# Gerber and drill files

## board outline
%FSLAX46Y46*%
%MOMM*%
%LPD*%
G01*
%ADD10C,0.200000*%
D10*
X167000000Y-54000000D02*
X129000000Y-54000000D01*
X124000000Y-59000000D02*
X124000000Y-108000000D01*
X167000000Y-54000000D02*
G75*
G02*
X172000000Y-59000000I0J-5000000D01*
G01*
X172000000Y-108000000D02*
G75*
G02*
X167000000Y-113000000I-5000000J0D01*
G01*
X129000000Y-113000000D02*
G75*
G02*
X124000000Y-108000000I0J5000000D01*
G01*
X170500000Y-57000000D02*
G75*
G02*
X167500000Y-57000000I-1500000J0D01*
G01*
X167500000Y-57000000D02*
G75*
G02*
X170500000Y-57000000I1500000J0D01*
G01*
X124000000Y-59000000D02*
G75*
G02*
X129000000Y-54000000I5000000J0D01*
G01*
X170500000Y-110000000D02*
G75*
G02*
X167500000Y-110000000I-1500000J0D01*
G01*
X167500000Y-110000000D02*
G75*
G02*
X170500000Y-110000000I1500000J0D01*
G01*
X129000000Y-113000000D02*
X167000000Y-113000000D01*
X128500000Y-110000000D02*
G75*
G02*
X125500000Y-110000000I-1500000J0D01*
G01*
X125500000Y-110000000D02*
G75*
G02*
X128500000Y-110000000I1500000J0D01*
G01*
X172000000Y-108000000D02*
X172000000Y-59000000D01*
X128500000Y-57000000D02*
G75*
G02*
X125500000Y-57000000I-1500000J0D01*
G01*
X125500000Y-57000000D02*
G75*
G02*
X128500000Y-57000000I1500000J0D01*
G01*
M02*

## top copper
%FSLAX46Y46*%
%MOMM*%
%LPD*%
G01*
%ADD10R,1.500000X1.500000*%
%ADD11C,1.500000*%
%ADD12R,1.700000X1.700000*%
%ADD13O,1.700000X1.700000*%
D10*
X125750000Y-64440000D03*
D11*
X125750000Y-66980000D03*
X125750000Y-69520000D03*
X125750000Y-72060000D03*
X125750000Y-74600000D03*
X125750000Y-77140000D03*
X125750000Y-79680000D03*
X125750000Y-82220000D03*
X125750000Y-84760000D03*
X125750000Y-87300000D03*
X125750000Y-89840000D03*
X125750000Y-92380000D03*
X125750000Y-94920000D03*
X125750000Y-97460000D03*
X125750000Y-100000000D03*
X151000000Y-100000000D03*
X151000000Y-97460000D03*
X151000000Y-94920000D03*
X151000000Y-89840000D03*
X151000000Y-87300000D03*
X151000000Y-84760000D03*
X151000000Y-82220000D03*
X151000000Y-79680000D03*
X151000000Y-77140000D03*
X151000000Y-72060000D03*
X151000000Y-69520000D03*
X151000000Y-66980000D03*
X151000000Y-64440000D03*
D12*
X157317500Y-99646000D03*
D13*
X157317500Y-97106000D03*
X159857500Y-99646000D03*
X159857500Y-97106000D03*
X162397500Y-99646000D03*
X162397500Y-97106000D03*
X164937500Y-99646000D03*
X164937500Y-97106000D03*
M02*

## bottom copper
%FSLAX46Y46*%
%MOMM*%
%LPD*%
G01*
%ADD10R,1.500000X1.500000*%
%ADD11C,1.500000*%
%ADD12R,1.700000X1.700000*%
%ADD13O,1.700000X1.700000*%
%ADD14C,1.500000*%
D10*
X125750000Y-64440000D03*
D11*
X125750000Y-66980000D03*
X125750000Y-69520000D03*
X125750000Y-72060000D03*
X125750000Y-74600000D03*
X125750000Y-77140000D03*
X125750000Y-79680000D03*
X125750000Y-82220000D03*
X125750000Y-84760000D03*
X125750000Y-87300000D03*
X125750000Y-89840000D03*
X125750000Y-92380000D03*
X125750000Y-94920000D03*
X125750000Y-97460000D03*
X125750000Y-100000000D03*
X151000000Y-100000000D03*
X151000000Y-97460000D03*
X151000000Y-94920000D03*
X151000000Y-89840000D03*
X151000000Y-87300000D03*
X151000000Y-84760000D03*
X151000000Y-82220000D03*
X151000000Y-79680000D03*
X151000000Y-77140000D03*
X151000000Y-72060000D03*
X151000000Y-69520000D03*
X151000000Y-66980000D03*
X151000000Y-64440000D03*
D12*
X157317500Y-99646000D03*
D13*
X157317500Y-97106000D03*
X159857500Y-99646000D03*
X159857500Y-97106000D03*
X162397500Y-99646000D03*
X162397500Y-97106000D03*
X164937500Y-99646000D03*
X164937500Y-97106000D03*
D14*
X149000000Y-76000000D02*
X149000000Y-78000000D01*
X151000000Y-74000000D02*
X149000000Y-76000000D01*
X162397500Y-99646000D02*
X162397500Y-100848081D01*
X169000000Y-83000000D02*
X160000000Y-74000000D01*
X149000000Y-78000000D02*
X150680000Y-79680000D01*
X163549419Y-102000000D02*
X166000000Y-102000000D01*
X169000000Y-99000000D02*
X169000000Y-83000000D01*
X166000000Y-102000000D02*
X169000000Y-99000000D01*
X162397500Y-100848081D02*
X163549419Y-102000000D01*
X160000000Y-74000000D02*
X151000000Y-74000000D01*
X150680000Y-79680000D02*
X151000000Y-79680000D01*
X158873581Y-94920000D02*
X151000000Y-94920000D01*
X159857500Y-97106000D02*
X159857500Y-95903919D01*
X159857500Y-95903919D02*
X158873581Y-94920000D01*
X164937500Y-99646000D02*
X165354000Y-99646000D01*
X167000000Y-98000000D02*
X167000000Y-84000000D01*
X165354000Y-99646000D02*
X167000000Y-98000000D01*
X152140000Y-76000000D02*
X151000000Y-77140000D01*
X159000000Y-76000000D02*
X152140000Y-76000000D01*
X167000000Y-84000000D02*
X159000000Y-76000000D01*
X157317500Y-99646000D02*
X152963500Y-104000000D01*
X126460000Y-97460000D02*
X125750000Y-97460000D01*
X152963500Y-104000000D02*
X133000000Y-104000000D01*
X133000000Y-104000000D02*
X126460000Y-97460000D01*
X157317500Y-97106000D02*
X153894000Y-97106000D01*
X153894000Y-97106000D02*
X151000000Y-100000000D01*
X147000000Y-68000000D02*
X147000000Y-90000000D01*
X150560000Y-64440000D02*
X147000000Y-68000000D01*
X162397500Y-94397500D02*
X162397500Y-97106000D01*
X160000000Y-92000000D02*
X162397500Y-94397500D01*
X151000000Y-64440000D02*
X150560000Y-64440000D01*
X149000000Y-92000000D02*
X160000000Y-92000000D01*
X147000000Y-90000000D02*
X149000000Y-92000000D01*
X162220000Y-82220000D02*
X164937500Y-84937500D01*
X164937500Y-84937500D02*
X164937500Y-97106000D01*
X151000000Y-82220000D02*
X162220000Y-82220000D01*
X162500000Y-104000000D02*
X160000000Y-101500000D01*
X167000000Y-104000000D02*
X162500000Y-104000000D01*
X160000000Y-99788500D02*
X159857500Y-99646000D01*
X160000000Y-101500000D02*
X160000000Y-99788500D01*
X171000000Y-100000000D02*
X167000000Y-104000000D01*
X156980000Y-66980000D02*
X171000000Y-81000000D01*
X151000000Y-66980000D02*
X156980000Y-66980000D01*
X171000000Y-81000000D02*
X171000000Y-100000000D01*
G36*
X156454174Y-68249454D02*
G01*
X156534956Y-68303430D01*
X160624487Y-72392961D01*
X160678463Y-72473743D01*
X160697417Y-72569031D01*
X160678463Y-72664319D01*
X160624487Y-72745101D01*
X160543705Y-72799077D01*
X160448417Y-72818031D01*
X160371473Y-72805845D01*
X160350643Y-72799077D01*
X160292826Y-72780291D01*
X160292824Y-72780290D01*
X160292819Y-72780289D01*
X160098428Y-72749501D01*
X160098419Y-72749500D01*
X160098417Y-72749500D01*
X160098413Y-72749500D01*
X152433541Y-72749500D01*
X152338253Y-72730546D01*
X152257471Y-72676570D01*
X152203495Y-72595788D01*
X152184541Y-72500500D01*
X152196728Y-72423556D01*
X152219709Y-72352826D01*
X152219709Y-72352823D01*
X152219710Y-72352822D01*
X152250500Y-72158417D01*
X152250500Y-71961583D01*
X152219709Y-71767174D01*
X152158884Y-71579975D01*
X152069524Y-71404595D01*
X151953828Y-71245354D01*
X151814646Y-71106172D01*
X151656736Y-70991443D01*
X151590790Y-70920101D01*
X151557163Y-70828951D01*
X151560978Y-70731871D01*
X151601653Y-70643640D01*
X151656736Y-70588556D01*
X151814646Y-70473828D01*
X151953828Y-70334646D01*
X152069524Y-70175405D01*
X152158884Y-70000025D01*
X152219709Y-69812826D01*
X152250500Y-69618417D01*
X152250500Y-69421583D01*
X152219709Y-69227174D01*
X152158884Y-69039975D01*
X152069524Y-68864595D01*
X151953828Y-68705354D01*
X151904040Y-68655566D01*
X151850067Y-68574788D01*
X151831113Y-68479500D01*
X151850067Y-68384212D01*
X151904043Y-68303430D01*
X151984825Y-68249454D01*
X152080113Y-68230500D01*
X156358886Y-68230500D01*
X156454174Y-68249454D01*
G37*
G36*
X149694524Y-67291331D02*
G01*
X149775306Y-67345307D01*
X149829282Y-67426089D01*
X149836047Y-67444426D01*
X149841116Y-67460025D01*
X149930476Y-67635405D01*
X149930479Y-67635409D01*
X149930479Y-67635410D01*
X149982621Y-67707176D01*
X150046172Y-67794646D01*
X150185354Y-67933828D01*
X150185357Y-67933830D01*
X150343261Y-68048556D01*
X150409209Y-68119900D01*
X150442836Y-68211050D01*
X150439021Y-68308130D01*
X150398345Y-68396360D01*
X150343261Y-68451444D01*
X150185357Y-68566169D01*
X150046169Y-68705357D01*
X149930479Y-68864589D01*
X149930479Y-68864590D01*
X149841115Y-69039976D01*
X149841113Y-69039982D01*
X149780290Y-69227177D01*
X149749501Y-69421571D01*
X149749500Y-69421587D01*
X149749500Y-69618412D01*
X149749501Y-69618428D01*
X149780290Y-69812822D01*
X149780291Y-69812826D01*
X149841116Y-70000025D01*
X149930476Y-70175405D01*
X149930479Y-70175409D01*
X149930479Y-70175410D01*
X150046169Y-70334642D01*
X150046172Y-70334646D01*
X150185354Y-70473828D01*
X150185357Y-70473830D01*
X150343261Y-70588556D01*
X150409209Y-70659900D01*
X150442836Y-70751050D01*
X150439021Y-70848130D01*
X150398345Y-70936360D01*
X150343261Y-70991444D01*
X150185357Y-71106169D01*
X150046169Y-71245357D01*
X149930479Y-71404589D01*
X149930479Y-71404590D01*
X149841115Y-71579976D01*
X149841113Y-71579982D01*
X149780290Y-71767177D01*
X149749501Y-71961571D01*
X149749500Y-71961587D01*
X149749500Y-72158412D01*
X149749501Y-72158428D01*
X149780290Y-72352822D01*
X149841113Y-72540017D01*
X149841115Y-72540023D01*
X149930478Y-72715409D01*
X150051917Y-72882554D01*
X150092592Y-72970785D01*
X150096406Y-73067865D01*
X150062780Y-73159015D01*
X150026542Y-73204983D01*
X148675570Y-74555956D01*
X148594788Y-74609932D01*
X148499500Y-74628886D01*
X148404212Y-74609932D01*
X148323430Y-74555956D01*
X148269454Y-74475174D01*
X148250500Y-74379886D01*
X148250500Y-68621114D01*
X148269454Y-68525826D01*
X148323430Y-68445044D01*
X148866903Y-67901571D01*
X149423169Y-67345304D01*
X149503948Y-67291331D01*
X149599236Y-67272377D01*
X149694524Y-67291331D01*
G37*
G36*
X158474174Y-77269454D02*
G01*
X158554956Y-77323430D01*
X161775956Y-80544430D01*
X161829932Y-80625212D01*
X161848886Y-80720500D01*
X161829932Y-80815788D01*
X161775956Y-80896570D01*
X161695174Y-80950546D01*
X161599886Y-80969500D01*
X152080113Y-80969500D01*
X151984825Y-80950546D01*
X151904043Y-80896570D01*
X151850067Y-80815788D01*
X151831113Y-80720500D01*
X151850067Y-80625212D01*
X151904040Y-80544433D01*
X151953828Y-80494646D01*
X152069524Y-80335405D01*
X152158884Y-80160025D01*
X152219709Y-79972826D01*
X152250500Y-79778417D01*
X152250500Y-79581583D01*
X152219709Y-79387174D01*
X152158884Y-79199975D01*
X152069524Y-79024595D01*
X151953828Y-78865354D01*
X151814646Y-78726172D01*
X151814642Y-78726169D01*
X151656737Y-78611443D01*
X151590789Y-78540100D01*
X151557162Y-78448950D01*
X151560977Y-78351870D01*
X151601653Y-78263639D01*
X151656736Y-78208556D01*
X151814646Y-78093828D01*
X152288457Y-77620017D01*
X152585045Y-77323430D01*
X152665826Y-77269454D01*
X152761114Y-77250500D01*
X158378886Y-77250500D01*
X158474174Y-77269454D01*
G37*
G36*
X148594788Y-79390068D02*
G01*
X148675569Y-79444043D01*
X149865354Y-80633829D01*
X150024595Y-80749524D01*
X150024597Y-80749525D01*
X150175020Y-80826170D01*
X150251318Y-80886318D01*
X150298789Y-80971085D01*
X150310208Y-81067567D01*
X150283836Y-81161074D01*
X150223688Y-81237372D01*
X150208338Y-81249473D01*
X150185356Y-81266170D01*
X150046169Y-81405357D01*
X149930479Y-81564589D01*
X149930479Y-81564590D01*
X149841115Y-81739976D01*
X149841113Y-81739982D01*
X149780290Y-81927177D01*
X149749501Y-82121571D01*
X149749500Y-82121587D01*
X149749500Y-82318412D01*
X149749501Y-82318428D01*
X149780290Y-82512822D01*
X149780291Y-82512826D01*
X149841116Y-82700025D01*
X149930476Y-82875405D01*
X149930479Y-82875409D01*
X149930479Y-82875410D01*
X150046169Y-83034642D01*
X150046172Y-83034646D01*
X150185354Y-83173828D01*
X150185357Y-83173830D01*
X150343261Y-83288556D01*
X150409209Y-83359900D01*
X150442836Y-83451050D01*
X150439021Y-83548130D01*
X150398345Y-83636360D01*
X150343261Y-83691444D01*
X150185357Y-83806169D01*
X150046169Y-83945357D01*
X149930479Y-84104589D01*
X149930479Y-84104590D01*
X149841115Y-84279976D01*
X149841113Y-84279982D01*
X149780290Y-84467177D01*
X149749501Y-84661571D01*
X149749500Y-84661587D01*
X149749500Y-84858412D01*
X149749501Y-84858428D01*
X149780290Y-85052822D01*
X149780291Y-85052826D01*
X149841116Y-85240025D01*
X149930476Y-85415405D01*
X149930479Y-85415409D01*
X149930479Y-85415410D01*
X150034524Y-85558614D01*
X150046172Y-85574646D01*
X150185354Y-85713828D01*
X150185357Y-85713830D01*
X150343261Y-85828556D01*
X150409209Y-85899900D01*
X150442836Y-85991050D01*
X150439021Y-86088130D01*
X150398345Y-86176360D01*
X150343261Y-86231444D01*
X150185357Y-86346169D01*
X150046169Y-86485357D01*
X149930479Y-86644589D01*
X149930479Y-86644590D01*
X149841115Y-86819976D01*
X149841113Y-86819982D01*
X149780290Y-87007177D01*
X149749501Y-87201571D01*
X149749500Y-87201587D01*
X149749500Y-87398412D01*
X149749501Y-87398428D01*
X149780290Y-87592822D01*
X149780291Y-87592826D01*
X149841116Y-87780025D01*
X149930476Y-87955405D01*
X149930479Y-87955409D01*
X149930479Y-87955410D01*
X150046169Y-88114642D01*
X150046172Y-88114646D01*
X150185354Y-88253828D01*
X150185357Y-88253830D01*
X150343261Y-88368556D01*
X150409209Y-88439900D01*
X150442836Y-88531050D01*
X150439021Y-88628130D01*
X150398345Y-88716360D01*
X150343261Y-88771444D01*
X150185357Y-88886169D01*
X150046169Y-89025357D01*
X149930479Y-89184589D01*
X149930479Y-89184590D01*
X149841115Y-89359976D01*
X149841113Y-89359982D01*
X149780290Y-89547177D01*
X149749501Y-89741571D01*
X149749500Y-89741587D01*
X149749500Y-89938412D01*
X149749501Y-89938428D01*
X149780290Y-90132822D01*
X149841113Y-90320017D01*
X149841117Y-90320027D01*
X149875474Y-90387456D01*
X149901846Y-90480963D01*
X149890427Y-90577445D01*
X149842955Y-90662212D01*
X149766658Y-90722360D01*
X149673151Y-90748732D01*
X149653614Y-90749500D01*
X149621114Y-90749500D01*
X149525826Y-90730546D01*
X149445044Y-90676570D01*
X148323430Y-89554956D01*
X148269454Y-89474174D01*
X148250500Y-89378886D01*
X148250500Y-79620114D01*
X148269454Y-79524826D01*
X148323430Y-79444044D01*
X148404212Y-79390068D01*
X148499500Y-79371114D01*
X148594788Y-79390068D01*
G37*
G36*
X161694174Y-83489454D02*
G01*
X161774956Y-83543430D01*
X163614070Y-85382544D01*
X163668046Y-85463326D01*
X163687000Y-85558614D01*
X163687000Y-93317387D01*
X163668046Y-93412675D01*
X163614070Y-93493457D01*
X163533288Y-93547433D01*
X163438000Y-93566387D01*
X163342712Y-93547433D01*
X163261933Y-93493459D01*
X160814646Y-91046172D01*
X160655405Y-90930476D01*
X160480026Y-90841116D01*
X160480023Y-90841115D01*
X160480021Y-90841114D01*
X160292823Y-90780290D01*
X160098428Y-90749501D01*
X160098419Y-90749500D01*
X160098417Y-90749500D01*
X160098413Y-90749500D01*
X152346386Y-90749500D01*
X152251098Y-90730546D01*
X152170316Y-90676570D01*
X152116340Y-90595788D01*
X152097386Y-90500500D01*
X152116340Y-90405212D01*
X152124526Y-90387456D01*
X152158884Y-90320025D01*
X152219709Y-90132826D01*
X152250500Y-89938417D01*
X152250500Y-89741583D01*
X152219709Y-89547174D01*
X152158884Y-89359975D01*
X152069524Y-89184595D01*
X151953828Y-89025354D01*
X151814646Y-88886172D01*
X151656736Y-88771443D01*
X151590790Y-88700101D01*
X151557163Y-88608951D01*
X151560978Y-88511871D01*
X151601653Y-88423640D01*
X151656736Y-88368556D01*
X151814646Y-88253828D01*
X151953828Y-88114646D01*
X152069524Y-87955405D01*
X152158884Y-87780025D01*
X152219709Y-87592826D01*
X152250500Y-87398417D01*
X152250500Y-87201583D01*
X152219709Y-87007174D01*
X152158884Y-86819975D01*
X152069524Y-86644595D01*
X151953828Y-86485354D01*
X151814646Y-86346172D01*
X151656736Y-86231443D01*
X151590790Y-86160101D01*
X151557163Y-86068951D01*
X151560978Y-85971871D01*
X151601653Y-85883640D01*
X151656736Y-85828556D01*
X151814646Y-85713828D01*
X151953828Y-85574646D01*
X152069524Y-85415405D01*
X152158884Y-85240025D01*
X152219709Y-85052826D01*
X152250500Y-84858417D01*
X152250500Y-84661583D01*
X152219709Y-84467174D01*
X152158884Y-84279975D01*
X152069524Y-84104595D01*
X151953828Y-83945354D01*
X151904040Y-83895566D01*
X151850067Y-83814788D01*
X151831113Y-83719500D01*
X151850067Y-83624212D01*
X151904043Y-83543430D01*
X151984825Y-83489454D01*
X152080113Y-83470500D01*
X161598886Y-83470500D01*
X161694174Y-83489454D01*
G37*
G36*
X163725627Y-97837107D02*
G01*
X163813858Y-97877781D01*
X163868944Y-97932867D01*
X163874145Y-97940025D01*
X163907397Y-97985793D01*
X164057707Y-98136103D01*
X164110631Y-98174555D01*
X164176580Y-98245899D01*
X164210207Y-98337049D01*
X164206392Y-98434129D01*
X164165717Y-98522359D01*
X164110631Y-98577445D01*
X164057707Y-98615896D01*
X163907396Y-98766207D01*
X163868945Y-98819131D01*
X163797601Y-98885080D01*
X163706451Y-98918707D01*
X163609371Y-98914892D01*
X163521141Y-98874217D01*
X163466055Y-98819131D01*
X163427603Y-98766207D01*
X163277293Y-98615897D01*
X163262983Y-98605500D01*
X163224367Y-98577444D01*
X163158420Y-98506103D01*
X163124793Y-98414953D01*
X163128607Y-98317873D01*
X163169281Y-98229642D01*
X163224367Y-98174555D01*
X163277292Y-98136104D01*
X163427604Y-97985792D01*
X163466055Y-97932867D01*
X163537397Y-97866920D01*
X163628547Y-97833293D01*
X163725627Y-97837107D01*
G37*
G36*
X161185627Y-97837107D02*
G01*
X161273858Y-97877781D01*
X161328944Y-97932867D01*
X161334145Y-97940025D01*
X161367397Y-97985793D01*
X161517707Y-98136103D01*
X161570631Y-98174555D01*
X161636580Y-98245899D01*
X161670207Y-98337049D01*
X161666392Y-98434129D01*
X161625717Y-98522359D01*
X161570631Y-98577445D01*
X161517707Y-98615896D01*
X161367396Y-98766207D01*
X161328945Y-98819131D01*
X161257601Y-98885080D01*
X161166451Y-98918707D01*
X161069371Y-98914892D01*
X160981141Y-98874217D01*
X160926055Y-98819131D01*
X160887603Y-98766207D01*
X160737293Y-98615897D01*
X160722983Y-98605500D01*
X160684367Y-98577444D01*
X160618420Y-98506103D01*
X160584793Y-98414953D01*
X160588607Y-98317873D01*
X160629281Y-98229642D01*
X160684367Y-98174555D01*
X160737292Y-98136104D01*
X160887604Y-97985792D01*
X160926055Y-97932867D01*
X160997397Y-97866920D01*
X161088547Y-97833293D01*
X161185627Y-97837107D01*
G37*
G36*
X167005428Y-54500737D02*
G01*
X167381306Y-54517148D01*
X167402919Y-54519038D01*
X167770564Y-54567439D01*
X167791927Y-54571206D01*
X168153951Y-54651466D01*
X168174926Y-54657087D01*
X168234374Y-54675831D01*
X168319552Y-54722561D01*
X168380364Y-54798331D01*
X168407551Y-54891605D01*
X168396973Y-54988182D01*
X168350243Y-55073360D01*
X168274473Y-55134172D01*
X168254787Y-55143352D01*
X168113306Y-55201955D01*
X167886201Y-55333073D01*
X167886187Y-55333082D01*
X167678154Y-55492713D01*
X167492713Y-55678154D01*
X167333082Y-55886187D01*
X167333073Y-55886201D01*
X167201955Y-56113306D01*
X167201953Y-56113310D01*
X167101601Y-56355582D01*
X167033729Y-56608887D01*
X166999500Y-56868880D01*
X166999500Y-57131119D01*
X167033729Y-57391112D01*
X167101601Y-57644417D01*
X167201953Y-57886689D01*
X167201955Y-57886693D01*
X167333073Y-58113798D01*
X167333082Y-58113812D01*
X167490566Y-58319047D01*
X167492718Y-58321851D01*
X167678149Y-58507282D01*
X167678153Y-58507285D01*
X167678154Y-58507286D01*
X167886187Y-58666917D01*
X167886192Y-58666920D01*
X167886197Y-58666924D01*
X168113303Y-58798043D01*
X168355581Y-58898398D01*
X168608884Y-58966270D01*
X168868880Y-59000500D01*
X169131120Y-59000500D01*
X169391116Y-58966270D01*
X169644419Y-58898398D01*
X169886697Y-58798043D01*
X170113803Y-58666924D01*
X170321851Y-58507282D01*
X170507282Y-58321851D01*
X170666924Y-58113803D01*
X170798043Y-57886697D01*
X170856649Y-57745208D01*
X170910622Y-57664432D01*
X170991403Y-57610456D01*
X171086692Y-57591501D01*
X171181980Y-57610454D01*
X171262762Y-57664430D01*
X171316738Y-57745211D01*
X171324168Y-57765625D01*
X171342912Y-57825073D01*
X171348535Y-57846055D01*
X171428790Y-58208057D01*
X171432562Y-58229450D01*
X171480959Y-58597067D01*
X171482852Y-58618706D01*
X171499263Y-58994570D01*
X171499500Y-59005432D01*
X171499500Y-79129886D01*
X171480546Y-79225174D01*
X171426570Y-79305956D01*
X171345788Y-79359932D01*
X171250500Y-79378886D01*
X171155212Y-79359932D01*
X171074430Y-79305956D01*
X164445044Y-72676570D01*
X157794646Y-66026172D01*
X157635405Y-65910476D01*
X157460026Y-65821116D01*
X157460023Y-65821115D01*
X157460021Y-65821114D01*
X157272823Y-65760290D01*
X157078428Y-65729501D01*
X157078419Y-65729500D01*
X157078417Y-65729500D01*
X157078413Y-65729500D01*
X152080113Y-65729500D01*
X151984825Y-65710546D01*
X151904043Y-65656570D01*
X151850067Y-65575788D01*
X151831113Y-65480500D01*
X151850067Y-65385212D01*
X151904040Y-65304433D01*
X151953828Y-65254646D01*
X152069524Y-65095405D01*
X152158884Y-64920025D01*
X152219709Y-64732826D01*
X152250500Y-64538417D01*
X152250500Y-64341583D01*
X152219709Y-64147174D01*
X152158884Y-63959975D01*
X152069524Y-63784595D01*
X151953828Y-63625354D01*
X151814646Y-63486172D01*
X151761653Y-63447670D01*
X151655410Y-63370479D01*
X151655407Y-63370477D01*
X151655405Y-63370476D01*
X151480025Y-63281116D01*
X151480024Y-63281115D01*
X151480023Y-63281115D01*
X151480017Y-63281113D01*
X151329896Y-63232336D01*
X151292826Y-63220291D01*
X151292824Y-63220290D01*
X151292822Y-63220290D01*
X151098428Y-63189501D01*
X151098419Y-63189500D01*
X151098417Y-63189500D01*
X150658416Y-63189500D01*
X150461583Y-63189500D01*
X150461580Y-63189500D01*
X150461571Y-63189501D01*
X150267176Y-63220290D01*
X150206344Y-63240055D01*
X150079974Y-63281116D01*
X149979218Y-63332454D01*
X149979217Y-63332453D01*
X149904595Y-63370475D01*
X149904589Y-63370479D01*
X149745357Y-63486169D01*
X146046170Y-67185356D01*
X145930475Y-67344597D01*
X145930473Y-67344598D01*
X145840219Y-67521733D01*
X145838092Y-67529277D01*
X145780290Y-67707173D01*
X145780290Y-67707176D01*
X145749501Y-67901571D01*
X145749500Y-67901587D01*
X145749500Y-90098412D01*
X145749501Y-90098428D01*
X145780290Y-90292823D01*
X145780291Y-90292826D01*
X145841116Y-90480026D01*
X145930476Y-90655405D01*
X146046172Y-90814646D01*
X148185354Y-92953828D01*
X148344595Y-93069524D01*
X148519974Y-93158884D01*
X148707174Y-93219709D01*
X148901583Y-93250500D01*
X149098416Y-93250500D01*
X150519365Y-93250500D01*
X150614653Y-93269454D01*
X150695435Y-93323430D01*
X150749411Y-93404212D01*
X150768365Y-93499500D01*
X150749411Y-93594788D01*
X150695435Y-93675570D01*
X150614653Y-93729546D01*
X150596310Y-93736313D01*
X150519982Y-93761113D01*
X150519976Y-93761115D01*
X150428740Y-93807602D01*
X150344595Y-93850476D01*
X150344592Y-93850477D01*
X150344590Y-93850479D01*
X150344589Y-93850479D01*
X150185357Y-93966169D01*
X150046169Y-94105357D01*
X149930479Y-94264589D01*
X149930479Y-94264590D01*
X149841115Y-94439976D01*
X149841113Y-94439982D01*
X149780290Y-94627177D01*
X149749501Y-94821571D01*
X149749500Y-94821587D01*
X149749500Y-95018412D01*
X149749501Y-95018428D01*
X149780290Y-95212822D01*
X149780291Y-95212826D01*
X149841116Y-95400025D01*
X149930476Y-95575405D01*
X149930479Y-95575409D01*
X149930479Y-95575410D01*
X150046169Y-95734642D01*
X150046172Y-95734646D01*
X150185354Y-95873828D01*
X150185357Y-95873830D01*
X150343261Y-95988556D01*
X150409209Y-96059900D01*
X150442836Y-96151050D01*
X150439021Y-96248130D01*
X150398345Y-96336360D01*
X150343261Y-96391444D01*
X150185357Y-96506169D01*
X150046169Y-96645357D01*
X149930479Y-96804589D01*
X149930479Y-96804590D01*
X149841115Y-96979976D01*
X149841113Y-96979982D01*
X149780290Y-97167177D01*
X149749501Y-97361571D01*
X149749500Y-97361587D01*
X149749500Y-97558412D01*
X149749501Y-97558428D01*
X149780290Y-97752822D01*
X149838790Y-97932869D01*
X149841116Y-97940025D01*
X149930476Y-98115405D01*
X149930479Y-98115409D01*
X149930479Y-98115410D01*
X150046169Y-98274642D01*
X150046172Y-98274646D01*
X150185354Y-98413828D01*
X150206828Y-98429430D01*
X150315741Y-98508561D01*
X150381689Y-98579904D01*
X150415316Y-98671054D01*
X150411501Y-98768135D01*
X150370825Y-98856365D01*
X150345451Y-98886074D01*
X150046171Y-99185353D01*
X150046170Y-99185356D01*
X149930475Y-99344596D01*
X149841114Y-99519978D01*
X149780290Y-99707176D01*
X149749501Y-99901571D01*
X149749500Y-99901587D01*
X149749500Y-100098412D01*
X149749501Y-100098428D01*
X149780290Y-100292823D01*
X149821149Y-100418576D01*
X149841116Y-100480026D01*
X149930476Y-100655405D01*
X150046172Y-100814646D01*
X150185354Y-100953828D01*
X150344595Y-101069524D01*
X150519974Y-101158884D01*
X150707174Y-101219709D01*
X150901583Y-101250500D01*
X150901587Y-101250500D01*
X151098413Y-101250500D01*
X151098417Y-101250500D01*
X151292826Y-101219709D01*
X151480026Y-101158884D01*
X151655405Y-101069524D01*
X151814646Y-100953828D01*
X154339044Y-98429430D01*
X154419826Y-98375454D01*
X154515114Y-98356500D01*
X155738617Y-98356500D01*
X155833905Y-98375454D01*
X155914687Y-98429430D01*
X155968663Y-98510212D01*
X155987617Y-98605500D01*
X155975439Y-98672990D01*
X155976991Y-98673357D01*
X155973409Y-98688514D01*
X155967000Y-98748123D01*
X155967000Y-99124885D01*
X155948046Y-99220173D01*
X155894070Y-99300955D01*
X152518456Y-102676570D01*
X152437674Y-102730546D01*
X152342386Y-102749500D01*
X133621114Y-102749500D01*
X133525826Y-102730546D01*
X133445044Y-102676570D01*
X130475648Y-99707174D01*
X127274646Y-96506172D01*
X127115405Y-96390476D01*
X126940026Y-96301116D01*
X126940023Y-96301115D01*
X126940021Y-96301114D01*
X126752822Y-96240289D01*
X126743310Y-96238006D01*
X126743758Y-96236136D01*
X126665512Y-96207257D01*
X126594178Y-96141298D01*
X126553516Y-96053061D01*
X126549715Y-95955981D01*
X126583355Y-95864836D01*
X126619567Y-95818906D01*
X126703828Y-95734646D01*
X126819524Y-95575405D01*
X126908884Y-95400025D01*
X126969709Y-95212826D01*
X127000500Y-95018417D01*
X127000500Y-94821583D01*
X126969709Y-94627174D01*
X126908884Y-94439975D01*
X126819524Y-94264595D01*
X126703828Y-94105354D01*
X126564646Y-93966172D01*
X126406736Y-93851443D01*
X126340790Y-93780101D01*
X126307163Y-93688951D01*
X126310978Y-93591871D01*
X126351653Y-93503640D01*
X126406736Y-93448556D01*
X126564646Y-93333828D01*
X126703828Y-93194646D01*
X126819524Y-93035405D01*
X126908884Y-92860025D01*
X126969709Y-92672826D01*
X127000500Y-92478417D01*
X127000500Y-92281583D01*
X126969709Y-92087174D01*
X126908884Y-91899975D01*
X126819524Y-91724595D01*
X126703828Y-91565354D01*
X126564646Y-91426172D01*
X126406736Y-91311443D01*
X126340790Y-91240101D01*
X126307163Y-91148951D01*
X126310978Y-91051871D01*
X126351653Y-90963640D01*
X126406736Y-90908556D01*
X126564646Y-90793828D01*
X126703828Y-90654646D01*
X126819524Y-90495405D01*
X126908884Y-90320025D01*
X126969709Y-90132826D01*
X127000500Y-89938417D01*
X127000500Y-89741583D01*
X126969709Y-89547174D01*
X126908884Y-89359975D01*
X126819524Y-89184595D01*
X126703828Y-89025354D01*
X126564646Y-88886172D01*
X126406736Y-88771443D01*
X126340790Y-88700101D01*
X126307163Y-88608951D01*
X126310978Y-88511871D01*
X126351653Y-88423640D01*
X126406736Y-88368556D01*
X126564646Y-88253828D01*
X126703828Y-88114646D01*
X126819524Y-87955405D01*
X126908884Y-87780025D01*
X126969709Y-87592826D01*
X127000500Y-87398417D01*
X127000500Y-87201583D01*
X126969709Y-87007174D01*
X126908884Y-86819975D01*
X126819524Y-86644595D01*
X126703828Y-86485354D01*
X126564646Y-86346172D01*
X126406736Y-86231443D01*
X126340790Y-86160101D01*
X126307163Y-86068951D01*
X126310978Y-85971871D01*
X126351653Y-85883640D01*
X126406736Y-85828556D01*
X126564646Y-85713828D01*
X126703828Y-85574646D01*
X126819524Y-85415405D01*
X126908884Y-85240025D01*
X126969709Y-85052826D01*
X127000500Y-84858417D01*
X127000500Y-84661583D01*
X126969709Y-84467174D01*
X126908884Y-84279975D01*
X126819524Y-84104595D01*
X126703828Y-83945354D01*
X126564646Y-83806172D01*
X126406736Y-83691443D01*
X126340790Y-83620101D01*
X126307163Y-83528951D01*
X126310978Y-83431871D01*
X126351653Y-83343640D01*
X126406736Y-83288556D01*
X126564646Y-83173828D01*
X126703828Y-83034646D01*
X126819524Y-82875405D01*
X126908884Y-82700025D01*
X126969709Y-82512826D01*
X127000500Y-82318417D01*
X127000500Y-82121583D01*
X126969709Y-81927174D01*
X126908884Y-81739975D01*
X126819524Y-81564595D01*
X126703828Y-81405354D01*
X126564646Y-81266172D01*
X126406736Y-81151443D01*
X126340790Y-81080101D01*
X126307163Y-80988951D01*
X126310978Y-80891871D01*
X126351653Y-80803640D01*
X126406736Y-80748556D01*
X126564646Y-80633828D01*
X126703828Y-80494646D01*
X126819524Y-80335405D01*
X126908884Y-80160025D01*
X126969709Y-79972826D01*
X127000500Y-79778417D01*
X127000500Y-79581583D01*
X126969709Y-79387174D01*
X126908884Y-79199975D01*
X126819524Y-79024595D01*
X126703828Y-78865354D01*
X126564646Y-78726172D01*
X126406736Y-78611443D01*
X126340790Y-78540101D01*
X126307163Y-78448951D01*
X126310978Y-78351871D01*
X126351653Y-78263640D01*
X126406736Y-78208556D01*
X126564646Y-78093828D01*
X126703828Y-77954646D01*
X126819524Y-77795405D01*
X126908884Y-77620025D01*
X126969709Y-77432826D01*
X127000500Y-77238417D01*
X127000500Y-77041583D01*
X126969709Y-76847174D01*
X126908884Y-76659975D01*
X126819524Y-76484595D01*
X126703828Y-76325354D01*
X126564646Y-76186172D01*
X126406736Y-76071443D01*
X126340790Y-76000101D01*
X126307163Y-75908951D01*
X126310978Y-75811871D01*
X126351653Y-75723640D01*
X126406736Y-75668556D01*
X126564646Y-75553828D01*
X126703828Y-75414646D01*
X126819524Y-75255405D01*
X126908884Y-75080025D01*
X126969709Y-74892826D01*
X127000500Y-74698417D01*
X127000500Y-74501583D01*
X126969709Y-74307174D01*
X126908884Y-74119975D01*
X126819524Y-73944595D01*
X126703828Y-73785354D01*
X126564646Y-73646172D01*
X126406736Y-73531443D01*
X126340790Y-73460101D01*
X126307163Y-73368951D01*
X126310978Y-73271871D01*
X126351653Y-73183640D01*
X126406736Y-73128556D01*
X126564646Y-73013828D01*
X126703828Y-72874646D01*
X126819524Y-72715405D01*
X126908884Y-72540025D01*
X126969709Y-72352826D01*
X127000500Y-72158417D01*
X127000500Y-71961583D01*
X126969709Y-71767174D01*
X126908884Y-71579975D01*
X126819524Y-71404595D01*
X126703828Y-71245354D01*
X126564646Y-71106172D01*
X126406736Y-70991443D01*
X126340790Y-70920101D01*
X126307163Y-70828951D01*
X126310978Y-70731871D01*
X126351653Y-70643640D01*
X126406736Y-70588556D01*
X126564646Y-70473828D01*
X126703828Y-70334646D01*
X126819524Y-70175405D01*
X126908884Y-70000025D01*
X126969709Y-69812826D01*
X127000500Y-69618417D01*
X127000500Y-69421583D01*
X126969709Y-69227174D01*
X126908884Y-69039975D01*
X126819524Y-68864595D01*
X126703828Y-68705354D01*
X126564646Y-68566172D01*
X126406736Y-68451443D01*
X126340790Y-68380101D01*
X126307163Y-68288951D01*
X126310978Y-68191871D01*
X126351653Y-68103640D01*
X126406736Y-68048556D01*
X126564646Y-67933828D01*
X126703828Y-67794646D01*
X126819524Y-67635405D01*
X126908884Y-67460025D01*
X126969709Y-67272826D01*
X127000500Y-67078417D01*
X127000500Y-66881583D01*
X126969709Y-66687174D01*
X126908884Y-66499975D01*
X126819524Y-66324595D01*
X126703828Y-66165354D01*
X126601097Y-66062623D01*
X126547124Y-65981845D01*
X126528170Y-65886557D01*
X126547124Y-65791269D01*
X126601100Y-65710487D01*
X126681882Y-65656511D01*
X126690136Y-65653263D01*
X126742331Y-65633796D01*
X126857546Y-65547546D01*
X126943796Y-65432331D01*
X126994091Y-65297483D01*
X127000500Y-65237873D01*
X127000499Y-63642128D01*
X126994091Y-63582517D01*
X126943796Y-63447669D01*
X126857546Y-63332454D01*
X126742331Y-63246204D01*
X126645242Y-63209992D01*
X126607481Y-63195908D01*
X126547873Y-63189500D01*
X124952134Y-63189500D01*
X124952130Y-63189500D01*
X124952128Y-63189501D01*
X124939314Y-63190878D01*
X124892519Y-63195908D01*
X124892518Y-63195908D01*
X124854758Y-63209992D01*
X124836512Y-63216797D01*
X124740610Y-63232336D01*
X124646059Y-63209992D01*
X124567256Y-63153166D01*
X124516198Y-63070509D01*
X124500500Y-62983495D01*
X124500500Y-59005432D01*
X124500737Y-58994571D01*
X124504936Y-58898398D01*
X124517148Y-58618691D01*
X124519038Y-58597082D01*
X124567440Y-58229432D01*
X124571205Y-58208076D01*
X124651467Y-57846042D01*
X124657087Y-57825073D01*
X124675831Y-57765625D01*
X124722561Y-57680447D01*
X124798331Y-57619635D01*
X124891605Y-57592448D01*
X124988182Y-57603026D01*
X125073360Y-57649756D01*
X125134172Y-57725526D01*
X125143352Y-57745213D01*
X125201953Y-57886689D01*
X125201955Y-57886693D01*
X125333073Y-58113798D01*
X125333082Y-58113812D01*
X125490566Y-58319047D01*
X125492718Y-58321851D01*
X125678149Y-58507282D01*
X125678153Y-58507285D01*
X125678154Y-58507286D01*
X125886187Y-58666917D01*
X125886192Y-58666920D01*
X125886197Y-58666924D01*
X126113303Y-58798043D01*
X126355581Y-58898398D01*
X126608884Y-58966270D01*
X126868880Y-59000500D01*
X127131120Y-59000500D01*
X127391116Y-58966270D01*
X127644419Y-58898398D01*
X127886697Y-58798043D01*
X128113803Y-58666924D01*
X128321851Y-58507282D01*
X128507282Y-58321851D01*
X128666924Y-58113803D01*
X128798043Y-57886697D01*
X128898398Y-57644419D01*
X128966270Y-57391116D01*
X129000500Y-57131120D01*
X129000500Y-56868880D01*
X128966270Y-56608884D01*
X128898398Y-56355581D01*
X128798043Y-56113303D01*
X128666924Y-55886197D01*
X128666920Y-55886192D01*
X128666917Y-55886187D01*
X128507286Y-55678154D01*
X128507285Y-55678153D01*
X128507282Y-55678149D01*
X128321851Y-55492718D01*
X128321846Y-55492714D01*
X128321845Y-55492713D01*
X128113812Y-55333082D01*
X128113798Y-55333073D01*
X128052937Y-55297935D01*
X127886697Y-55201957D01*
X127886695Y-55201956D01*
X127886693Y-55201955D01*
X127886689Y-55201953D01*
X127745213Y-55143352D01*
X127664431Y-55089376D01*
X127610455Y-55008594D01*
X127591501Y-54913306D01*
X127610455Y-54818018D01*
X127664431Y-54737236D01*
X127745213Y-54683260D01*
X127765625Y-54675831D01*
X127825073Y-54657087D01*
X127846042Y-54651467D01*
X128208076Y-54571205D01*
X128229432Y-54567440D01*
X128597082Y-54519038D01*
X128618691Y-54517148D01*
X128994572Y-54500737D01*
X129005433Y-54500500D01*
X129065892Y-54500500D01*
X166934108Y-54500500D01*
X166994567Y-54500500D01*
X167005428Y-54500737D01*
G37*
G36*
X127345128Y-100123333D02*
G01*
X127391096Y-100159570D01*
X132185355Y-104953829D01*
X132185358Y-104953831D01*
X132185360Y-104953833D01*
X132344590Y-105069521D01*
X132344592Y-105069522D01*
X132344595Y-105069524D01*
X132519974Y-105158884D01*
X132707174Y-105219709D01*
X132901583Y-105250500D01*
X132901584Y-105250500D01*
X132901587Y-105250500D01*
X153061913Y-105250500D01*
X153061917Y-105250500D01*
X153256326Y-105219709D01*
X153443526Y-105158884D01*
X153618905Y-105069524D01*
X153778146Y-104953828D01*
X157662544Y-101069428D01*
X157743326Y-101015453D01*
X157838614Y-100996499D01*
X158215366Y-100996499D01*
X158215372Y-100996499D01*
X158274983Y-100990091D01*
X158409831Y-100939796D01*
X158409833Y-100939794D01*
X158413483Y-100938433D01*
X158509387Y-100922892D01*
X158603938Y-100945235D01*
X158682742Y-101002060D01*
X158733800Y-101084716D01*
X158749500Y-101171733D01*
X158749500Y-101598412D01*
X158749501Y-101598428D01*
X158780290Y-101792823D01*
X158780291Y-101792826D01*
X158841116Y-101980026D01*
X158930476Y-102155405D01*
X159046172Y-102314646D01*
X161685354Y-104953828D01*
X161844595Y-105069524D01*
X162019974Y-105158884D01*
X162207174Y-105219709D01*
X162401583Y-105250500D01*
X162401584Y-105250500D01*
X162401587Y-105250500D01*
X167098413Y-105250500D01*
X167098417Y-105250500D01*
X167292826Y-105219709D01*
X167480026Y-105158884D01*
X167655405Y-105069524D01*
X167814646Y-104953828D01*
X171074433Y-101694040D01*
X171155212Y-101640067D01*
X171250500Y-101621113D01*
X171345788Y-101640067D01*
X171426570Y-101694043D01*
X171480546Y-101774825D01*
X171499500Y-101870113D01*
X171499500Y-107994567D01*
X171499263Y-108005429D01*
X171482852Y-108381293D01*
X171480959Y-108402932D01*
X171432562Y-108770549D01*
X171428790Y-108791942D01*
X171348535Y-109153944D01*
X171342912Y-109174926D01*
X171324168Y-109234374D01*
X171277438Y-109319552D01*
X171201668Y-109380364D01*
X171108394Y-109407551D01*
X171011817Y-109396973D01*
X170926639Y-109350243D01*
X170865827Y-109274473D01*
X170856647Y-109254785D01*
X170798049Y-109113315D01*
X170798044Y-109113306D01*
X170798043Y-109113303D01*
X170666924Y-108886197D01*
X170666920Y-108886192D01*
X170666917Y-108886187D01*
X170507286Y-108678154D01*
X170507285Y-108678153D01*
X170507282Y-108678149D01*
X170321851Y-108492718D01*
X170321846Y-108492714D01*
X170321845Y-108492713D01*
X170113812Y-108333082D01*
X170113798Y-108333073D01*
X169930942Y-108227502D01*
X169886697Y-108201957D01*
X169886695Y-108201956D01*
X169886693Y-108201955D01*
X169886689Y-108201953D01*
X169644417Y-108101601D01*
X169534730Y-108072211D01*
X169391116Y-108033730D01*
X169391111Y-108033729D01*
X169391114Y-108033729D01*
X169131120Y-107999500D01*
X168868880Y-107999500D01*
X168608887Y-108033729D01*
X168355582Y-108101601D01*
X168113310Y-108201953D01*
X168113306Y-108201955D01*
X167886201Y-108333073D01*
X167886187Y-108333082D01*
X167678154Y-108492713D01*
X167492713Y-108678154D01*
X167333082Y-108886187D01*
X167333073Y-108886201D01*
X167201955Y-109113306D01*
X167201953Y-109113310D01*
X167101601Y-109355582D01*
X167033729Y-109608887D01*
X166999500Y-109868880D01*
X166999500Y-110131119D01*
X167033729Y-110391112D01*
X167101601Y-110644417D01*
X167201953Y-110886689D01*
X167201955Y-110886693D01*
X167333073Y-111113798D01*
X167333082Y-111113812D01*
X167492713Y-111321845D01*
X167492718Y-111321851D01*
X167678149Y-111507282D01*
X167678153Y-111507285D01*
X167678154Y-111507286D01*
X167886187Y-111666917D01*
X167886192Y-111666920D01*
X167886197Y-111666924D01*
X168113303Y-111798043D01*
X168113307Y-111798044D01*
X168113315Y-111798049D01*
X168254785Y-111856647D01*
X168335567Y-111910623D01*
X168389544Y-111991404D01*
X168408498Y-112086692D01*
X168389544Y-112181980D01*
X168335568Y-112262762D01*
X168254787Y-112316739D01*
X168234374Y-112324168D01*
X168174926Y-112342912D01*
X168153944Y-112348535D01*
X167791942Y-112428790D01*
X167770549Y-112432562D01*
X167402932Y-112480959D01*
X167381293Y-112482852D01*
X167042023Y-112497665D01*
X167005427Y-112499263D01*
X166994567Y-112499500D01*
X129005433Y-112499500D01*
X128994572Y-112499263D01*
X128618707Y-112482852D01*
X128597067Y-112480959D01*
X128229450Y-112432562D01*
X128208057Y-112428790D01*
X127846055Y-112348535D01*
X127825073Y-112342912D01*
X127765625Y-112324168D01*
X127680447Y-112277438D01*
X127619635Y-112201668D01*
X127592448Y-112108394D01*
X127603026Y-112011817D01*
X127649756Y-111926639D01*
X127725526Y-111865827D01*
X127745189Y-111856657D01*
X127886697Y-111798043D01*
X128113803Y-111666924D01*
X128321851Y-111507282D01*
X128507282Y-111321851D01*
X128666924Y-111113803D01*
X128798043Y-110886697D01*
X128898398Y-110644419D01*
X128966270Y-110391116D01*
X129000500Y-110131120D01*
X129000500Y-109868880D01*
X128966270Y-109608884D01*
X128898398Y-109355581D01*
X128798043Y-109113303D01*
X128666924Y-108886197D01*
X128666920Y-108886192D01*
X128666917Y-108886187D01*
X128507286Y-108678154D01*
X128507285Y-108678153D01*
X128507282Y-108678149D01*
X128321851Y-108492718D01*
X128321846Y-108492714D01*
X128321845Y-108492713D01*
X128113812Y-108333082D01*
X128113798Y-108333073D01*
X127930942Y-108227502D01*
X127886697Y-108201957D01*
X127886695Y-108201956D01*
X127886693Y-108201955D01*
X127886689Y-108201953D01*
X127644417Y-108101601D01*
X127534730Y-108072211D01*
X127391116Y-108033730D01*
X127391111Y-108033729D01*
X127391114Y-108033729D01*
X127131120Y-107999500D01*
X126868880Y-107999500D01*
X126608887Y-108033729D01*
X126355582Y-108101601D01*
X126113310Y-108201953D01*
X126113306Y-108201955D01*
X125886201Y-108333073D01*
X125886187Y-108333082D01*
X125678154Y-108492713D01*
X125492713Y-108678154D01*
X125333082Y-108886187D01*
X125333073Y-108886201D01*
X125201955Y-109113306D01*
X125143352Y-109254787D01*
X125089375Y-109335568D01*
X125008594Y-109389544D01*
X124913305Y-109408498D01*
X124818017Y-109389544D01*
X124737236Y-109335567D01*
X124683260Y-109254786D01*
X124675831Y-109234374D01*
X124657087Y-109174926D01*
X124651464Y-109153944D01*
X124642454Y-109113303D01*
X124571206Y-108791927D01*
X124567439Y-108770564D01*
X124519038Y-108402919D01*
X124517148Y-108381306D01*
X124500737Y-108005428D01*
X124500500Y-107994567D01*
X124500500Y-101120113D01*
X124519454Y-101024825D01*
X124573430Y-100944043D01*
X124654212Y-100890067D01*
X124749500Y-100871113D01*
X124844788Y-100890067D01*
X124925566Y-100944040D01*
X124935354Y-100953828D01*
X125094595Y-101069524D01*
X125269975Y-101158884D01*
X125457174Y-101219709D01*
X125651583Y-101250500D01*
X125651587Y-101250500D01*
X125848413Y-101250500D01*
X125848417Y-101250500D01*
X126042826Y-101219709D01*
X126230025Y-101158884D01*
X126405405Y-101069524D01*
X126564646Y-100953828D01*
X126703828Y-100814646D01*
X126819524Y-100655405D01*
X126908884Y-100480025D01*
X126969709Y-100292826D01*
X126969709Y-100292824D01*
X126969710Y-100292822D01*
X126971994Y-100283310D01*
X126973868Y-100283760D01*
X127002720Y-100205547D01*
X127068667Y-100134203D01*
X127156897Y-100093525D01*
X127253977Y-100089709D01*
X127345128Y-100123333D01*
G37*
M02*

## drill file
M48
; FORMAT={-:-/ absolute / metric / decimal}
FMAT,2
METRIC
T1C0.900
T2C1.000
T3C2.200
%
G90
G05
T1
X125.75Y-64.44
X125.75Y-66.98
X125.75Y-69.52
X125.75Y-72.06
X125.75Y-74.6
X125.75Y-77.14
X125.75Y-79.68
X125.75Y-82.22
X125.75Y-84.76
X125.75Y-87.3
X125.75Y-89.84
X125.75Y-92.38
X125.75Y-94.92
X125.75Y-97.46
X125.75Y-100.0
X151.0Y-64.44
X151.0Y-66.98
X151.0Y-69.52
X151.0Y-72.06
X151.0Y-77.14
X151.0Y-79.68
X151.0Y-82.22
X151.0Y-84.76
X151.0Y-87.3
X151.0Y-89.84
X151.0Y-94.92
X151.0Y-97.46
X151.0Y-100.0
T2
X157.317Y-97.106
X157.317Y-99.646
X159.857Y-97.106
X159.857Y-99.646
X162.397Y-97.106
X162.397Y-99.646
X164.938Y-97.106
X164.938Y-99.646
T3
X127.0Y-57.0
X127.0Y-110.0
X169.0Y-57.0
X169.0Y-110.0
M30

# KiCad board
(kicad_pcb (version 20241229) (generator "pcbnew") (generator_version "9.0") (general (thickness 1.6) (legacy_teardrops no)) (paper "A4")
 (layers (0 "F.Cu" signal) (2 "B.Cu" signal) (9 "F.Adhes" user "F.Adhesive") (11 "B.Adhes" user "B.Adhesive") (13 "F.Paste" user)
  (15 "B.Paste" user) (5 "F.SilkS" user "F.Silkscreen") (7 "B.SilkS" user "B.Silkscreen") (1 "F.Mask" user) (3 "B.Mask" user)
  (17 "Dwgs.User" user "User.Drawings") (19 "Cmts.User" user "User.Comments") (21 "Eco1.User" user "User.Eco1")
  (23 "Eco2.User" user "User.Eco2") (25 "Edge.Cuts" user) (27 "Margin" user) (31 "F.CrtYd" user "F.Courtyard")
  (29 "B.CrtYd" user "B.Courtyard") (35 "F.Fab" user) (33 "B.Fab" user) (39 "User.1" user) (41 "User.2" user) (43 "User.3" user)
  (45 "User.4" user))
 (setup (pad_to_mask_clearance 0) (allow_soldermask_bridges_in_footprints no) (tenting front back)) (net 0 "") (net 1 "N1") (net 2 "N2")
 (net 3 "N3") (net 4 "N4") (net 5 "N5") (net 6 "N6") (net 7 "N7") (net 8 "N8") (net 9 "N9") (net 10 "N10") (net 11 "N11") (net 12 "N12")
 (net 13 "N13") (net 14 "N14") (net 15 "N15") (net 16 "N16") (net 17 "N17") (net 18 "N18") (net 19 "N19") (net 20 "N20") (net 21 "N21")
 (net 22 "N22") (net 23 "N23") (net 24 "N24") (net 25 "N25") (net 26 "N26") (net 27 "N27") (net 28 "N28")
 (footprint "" (layer "F.Cu") (at 169 110)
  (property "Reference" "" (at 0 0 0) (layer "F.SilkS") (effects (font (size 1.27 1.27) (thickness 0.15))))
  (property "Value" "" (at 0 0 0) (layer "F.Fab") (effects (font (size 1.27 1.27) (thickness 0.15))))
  (pad "" np_thru_hole circle (at 0 0) (size 2.2 2.2) (drill 2.2) (layers "*.Cu" "*.Mask")))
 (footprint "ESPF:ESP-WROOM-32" (layer "F.Cu") (at 121.3175 102.714)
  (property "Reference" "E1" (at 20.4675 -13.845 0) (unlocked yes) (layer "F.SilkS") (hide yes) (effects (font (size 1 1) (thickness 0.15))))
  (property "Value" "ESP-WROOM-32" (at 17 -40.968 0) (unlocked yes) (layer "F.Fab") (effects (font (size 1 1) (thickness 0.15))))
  (pad "1" thru_hole rect (at 4.4325 -38.274) (size 1.5 1.5) (drill 0.9) (layers "*.Cu" "*.Mask") (remove_unused_layers yes)
   (keep_end_layers yes) (zone_layer_connections) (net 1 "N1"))
  (pad "2" thru_hole circle (at 4.4325 -35.734) (size 1.5 1.5) (drill 0.9) (layers "*.Cu" "*.Mask") (remove_unused_layers yes)
   (keep_end_layers yes) (zone_layer_connections) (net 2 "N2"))
  (pad "3" thru_hole circle (at 4.4325 -33.194) (size 1.5 1.5) (drill 0.9) (layers "*.Cu" "*.Mask") (remove_unused_layers yes)
   (keep_end_layers yes) (zone_layer_connections) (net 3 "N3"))
  (pad "4" thru_hole circle (at 4.4325 -30.654) (size 1.5 1.5) (drill 0.9) (layers "*.Cu" "*.Mask") (remove_unused_layers yes)
   (keep_end_layers yes) (zone_layer_connections) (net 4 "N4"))
  (pad "5" thru_hole circle (at 4.4325 -28.114) (size 1.5 1.5) (drill 0.9) (layers "*.Cu" "*.Mask") (remove_unused_layers yes)
   (keep_end_layers yes) (zone_layer_connections) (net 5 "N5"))
  (pad "6" thru_hole circle (at 4.4325 -25.574) (size 1.5 1.5) (drill 0.9) (layers "*.Cu" "*.Mask") (remove_unused_layers yes)
   (keep_end_layers yes) (zone_layer_connections) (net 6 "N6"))
  (pad "7" thru_hole circle (at 4.4325 -23.034) (size 1.5 1.5) (drill 0.9) (layers "*.Cu" "*.Mask") (remove_unused_layers yes)
   (keep_end_layers yes) (zone_layer_connections) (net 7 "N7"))
  (pad "8" thru_hole circle (at 4.4325 -20.494) (size 1.5 1.5) (drill 0.9) (layers "*.Cu" "*.Mask") (remove_unused_layers yes)
   (keep_end_layers yes) (zone_layer_connections) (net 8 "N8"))
  (pad "9" thru_hole circle (at 4.4325 -17.954) (size 1.5 1.5) (drill 0.9) (layers "*.Cu" "*.Mask") (remove_unused_layers yes)
   (keep_end_layers yes) (zone_layer_connections) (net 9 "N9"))
  (pad "10" thru_hole circle (at 4.4325 -15.414) (size 1.5 1.5) (drill 0.9) (layers "*.Cu" "*.Mask") (remove_unused_layers yes)
   (keep_end_layers yes) (zone_layer_connections) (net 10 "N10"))
  (pad "11" thru_hole circle (at 4.4325 -12.874) (size 1.5 1.5) (drill 0.9) (layers "*.Cu" "*.Mask") (remove_unused_layers yes)
   (keep_end_layers yes) (zone_layer_connections) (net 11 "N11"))
  (pad "12" thru_hole circle (at 4.4325 -10.334) (size 1.5 1.5) (drill 0.9) (layers "*.Cu" "*.Mask") (remove_unused_layers yes)
   (keep_end_layers yes) (zone_layer_connections) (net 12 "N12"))
  (pad "13" thru_hole circle (at 4.4325 -7.794) (size 1.5 1.5) (drill 0.9) (layers "*.Cu" "*.Mask") (remove_unused_layers yes)
   (keep_end_layers yes) (zone_layer_connections) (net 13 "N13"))
  (pad "14" thru_hole circle (at 4.4325 -5.254) (size 1.5 1.5) (drill 0.9) (layers "*.Cu" "*.Mask") (remove_unused_layers yes)
   (keep_end_layers yes) (zone_layer_connections) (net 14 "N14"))
  (pad "15" thru_hole circle (at 4.4325 -2.714) (size 1.5 1.5) (drill 0.9) (layers "*.Cu" "*.Mask") (remove_unused_layers yes)
   (keep_end_layers yes) (zone_layer_connections) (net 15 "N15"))
  (pad "16" thru_hole circle (at 29.6825 -2.714) (size 1.5 1.5) (drill 0.9) (layers "*.Cu" "*.Mask") (remove_unused_layers yes)
   (keep_end_layers yes) (zone_layer_connections) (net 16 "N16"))
  (pad "17" thru_hole circle (at 29.6825 -5.254) (size 1.5 1.5) (drill 0.9) (layers "*.Cu" "*.Mask") (remove_unused_layers yes)
   (keep_end_layers yes) (zone_layer_connections) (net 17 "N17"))
  (pad "18" thru_hole circle (at 29.6825 -7.794) (size 1.5 1.5) (drill 0.9) (layers "*.Cu" "*.Mask") (remove_unused_layers yes)
   (keep_end_layers yes) (zone_layer_connections) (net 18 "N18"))
  (pad "20" thru_hole circle (at 29.6825 -12.874) (size 1.5 1.5) (drill 0.9) (layers "*.Cu" "*.Mask") (remove_unused_layers yes)
   (keep_end_layers yes) (zone_layer_connections) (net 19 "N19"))
  (pad "21" thru_hole circle (at 29.6825 -15.414) (size 1.5 1.5) (drill 0.9) (layers "*.Cu" "*.Mask") (remove_unused_layers yes)
   (keep_end_layers yes) (zone_layer_connections) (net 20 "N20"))
  (pad "22" thru_hole circle (at 29.6825 -17.954) (size 1.5 1.5) (drill 0.9) (layers "*.Cu" "*.Mask") (remove_unused_layers yes)
   (keep_end_layers yes) (zone_layer_connections) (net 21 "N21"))
  (pad "23" thru_hole circle (at 29.6825 -20.494) (size 1.5 1.5) (drill 0.9) (layers "*.Cu" "*.Mask") (remove_unused_layers yes)
   (keep_end_layers yes) (zone_layer_connections) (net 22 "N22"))
  (pad "24" thru_hole circle (at 29.6825 -23.034) (size 1.5 1.5) (drill 0.9) (layers "*.Cu" "*.Mask") (remove_unused_layers yes)
   (keep_end_layers yes) (zone_layer_connections) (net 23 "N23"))
  (pad "25" thru_hole circle (at 29.6825 -25.574) (size 1.5 1.5) (drill 0.9) (layers "*.Cu" "*.Mask") (remove_unused_layers yes)
   (keep_end_layers yes) (zone_layer_connections) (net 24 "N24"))
  (pad "27" thru_hole circle (at 29.6825 -30.654) (size 1.5 1.5) (drill 0.9) (layers "*.Cu" "*.Mask") (remove_unused_layers yes)
   (keep_end_layers yes) (zone_layer_connections) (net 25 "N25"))
  (pad "28" thru_hole circle (at 29.6825 -33.194) (size 1.5 1.5) (drill 0.9) (layers "*.Cu" "*.Mask") (remove_unused_layers yes)
   (keep_end_layers yes) (zone_layer_connections) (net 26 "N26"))
  (pad "29" thru_hole circle (at 29.6825 -35.734) (size 1.5 1.5) (drill 0.9) (layers "*.Cu" "*.Mask") (remove_unused_layers yes)
   (keep_end_layers yes) (zone_layer_connections) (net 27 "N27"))
  (pad "30" thru_hole circle (at 29.6825 -38.274) (size 1.5 1.5) (drill 0.9) (layers "*.Cu" "*.Mask") (remove_unused_layers yes)
   (keep_end_layers yes) (zone_layer_connections) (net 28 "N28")))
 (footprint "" (layer "F.Cu") (at 127 110)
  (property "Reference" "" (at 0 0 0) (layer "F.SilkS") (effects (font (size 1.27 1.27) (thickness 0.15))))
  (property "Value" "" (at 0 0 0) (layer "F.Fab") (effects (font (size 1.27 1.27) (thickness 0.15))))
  (pad "" np_thru_hole circle (at 0 0) (size 2.2 2.2) (drill 2.2) (layers "*.Cu" "*.Mask")))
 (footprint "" (layer "F.Cu") (at 127 57)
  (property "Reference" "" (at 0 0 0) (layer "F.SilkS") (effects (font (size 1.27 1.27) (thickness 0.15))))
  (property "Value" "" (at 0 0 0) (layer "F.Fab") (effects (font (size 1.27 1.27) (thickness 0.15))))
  (pad "" np_thru_hole circle (at 0 0) (size 2.2 2.2) (drill 2.2) (layers "*.Cu" "*.Mask")))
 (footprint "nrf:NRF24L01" (layer "F.Cu") (at 174.2805 103.331 90)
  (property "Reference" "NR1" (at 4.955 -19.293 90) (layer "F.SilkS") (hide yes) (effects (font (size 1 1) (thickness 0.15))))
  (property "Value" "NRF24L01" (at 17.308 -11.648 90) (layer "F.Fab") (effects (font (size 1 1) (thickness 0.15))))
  (pad "1" thru_hole rect (at 3.685 -16.963 90) (size 1.7 1.7) (drill 1) (layers "*.Cu" "*.Mask") (remove_unused_layers no) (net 14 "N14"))
  (pad "2" thru_hole oval (at 6.225 -16.963 90) (size 1.7 1.7) (drill 1) (layers "*.Cu" "*.Mask") (remove_unused_layers no) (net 16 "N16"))
  (pad "3" thru_hole oval (at 3.685 -14.423 90) (size 1.7 1.7) (drill 1) (layers "*.Cu" "*.Mask") (remove_unused_layers no) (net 27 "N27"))
  (pad "4" thru_hole oval (at 6.225 -14.423 90) (size 1.7 1.7) (drill 1) (layers "*.Cu" "*.Mask") (remove_unused_layers no) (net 18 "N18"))
  (pad "5" thru_hole oval (at 3.685 -11.883 90) (size 1.7 1.7) (drill 1) (layers "*.Cu" "*.Mask") (remove_unused_layers no) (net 23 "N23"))
  (pad "6" thru_hole oval (at 6.225 -11.883 90) (size 1.7 1.7) (drill 1) (layers "*.Cu" "*.Mask") (remove_unused_layers no) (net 28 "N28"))
  (pad "7" thru_hole oval (at 3.685 -9.343 90) (size 1.7 1.7) (drill 1) (layers "*.Cu" "*.Mask") (remove_unused_layers no) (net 24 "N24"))
  (pad "8" thru_hole oval (at 6.225 -9.343 90) (size 1.7 1.7) (drill 1) (layers "*.Cu" "*.Mask") (remove_unused_layers no) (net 22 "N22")))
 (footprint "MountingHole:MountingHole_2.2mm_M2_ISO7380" (layer "F.Cu") (at 169 57)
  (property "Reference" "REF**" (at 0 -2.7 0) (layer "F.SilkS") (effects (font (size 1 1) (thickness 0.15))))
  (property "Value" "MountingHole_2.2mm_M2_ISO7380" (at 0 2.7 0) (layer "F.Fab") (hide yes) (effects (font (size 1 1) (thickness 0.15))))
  (pad "" np_thru_hole circle (at 0 0) (size 2.2 2.2) (drill 2.2) (layers "*.Cu" "*.Mask")))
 (gr_line (start 167 54) (end 129 54) (stroke (width 0.2) (type default)) (layer "Edge.Cuts"))
 (gr_line (start 124 59) (end 124 108) (stroke (width 0.2) (type default)) (layer "Edge.Cuts"))
 (gr_arc (start 167 54) (mid 170.535534 55.464466) (end 172 59) (stroke (width 0.2) (type default)) (layer "Edge.Cuts"))
 (gr_arc (start 172 108) (mid 170.535534 111.535534) (end 167 113) (stroke (width 0.2) (type default)) (layer "Edge.Cuts"))
 (gr_arc (start 129 113) (mid 125.464466 111.535534) (end 124 108) (stroke (width 0.2) (type default)) (layer "Edge.Cuts"))
 (gr_circle (center 169 57) (end 170.5 57) (stroke (width 0.2) (type default)) (fill no) (layer "Edge.Cuts"))
 (gr_arc (start 124 59) (mid 125.464466 55.464466) (end 129 54) (stroke (width 0.2) (type default)) (layer "Edge.Cuts"))
 (gr_circle (center 169 110) (end 170.5 110) (stroke (width 0.2) (type default)) (fill no) (layer "Edge.Cuts"))
 (gr_line (start 129 113) (end 167 113) (stroke (width 0.2) (type default)) (layer "Edge.Cuts"))
 (gr_circle (center 127 110) (end 128.5 110) (stroke (width 0.2) (type default)) (fill no) (layer "Edge.Cuts"))
 (gr_line (start 172 108) (end 172 59) (stroke (width 0.2) (type default)) (layer "Edge.Cuts"))
 (gr_circle (center 127 57) (end 128.5 57) (stroke (width 0.2) (type default)) (fill no) (layer "Edge.Cuts"))
 (segment (start 149 76) (end 149 78) (width 1.5) (layer "B.Cu") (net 23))
 (segment (start 151 74) (end 149 76) (width 1.5) (layer "B.Cu") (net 23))
 (segment (start 162.3975 99.646) (end 162.3975 100.848081) (width 1.5) (layer "B.Cu") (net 23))
 (segment (start 169 83) (end 160 74) (width 1.5) (layer "B.Cu") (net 23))
 (segment (start 149 78) (end 150.68 79.68) (width 1.5) (layer "B.Cu") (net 23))
 (segment (start 163.549419 102) (end 166 102) (width 1.5) (layer "B.Cu") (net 23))
 (segment (start 169 99) (end 169 83) (width 1.5) (layer "B.Cu") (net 23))
 (segment (start 166 102) (end 169 99) (width 1.5) (layer "B.Cu") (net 23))
 (segment (start 162.3975 100.848081) (end 163.549419 102) (width 1.5) (layer "B.Cu") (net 23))
 (segment (start 160 74) (end 151 74) (width 1.5) (layer "B.Cu") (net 23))
 (segment (start 150.68 79.68) (end 151 79.68) (width 1.5) (layer "B.Cu") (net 23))
 (segment (start 158.873581 94.92) (end 151 94.92) (width 1.5) (layer "B.Cu") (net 18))
 (segment (start 159.8575 97.106) (end 159.8575 95.903919) (width 1.5) (layer "B.Cu") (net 18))
 (segment (start 159.8575 95.903919) (end 158.873581 94.92) (width 1.5) (layer "B.Cu") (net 18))
 (segment (start 164.9375 99.646) (end 165.354 99.646) (width 1.5) (layer "B.Cu") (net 24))
 (segment (start 167 98) (end 167 84) (width 1.5) (layer "B.Cu") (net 24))
 (segment (start 165.354 99.646) (end 167 98) (width 1.5) (layer "B.Cu") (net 24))
 (segment (start 152.14 76) (end 151 77.14) (width 1.5) (layer "B.Cu") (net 24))
 (segment (start 159 76) (end 152.14 76) (width 1.5) (layer "B.Cu") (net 24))
 (segment (start 167 84) (end 159 76) (width 1.5) (layer "B.Cu") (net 24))
 (segment (start 157.3175 99.646) (end 152.9635 104) (width 1.5) (layer "B.Cu") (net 14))
 (segment (start 126.46 97.46) (end 125.75 97.46) (width 1.5) (layer "B.Cu") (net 14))
 (segment (start 152.9635 104) (end 133 104) (width 1.5) (layer "B.Cu") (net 14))
 (segment (start 133 104) (end 126.46 97.46) (width 1.5) (layer "B.Cu") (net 14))
 (segment (start 157.3175 97.106) (end 153.894 97.106) (width 1.5) (layer "B.Cu") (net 16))
 (segment (start 153.894 97.106) (end 151 100) (width 1.5) (layer "B.Cu") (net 16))
 (segment (start 147 68) (end 147 90) (width 1.5) (layer "B.Cu") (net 28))
 (segment (start 150.56 64.44) (end 147 68) (width 1.5) (layer "B.Cu") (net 28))
 (segment (start 162.3975 94.3975) (end 162.3975 97.106) (width 1.5) (layer "B.Cu") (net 28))
 (segment (start 160 92) (end 162.3975 94.3975) (width 1.5) (layer "B.Cu") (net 28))
 (segment (start 151 64.44) (end 150.56 64.44) (width 1.5) (layer "B.Cu") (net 28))
 (segment (start 149 92) (end 160 92) (width 1.5) (layer "B.Cu") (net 28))
 (segment (start 147 90) (end 149 92) (width 1.5) (layer "B.Cu") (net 28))
 (segment (start 162.22 82.22) (end 164.9375 84.9375) (width 1.5) (layer "B.Cu") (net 22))
 (segment (start 164.9375 84.9375) (end 164.9375 97.106) (width 1.5) (layer "B.Cu") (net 22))
 (segment (start 151 82.22) (end 162.22 82.22) (width 1.5) (layer "B.Cu") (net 22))
 (segment (start 162.5 104) (end 160 101.5) (width 1.5) (layer "B.Cu") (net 27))
 (segment (start 167 104) (end 162.5 104) (width 1.5) (layer "B.Cu") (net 27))
 (segment (start 160 99.7885) (end 159.8575 99.646) (width 1.5) (layer "B.Cu") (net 27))
 (segment (start 160 101.5) (end 160 99.7885) (width 1.5) (layer "B.Cu") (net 27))
 (segment (start 171 100) (end 167 104) (width 1.5) (layer "B.Cu") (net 27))
 (segment (start 156.98 66.98) (end 171 81) (width 1.5) (layer "B.Cu") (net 27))
 (segment (start 151 66.98) (end 156.98 66.98) (width 1.5) (layer "B.Cu") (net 27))
 (segment (start 171 81) (end 171 100) (width 1.5) (layer "B.Cu") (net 27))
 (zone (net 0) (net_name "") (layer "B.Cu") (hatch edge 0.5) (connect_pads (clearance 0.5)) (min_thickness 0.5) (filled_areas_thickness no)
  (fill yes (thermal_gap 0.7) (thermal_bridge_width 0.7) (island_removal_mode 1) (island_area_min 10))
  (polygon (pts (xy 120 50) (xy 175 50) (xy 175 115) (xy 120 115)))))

